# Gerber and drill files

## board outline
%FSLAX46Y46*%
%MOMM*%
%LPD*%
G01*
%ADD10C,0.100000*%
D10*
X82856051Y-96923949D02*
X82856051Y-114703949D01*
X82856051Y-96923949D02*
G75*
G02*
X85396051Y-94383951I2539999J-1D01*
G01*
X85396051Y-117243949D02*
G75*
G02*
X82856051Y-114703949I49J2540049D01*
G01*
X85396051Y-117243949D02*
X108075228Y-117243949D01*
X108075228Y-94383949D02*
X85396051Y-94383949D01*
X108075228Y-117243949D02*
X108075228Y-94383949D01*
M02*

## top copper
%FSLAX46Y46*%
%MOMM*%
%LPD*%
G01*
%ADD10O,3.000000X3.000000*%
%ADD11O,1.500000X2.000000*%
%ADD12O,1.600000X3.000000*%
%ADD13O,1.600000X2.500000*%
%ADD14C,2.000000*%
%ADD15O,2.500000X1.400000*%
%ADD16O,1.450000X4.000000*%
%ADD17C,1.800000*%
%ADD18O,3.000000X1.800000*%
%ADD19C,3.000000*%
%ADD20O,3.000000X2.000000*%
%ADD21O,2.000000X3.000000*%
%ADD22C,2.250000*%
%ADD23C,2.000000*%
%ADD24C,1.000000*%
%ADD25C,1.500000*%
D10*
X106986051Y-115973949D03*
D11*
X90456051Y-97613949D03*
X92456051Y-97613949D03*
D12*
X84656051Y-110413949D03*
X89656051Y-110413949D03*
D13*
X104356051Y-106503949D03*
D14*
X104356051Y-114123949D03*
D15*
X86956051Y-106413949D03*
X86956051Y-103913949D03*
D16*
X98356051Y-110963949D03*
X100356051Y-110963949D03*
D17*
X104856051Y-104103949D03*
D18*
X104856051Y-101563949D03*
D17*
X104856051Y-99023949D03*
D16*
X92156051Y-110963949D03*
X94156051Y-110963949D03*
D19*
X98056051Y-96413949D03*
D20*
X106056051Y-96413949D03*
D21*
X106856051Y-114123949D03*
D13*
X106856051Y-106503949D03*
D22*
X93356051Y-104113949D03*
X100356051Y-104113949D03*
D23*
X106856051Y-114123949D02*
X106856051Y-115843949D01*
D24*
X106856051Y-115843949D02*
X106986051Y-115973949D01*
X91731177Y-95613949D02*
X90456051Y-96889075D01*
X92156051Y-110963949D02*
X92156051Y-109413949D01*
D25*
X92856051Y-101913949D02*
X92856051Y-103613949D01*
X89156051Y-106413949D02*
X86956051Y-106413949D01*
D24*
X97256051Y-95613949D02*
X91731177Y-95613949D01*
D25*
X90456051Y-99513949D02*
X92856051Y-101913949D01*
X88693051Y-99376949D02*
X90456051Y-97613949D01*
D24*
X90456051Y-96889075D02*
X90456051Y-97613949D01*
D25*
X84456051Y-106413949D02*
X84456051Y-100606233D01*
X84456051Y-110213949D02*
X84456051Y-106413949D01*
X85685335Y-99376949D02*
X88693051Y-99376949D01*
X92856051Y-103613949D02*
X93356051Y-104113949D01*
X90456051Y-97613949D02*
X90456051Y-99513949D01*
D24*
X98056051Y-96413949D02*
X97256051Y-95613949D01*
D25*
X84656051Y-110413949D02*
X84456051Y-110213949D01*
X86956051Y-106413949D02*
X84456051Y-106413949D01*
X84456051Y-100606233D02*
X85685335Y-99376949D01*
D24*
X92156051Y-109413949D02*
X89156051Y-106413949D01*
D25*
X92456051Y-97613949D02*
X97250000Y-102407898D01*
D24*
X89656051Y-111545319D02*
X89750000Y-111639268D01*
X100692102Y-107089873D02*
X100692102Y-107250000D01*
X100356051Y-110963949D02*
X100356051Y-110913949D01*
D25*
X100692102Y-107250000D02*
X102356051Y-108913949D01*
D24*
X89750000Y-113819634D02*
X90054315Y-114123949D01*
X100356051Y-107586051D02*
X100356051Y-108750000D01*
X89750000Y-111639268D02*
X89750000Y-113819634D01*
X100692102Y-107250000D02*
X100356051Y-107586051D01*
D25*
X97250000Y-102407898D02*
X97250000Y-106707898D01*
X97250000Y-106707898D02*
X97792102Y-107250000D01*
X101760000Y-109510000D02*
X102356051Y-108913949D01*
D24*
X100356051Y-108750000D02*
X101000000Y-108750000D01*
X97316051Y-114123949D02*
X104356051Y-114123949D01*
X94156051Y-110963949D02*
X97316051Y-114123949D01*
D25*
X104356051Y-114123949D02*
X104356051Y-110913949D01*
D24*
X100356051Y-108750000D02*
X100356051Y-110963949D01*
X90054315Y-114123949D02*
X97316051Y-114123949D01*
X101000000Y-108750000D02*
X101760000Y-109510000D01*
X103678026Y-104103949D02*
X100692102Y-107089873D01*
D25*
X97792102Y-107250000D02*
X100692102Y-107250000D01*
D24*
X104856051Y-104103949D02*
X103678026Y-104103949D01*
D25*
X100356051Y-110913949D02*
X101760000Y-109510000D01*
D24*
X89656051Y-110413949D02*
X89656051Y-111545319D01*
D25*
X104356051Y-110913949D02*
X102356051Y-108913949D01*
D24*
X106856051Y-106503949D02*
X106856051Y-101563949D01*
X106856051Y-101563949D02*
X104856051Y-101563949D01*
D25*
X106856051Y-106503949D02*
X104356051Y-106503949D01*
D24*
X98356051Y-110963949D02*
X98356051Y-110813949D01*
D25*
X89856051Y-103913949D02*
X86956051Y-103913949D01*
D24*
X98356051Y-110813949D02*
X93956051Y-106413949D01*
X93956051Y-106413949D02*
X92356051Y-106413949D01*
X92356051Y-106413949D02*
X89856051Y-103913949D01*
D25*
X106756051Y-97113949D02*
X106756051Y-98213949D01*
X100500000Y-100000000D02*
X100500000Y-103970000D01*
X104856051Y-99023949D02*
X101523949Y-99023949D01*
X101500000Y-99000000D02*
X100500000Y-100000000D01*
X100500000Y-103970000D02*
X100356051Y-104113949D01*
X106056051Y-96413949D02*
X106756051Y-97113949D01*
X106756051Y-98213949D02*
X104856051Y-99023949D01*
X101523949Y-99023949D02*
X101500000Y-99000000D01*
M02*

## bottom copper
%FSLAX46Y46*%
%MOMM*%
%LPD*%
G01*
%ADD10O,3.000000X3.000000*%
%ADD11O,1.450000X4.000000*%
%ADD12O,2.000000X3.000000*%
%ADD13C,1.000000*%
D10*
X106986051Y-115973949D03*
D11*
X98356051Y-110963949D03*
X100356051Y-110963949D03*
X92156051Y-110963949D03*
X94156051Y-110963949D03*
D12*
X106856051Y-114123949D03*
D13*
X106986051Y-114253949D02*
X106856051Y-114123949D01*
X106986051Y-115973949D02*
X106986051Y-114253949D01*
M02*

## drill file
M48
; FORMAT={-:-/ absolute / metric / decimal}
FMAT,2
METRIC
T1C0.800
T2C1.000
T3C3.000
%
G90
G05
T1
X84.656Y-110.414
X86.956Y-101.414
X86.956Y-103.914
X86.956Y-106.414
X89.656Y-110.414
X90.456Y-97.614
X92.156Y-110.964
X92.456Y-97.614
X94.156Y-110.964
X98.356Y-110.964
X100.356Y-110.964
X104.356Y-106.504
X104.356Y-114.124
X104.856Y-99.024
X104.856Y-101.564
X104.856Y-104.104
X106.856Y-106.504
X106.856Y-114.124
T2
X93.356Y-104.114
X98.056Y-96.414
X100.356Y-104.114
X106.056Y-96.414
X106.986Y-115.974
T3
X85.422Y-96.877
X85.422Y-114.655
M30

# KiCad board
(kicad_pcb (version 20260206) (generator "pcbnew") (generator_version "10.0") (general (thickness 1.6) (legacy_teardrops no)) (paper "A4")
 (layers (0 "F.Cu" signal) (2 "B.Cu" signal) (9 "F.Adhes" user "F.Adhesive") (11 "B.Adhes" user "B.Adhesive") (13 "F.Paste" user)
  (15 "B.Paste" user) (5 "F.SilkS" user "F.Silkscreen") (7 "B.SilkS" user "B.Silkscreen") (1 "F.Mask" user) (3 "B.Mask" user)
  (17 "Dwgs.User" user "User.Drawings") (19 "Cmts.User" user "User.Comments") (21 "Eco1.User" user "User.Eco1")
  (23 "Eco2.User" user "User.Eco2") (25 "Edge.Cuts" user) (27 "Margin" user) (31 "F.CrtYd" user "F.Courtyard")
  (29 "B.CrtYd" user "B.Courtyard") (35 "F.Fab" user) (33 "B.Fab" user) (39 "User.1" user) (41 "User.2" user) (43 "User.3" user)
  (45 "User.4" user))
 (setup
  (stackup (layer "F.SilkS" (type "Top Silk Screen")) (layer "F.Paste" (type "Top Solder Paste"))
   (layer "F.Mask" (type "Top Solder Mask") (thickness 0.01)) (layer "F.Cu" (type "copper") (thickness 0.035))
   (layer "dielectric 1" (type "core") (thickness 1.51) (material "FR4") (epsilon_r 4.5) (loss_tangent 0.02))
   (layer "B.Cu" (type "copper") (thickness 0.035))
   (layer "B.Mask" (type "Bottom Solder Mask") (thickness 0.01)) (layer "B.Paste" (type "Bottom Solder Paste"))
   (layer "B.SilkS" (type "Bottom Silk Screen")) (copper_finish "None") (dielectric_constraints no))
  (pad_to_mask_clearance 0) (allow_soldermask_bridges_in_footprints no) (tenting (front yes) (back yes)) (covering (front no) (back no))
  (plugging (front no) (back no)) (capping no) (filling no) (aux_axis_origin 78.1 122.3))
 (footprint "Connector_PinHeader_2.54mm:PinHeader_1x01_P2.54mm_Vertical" (layer "F.Cu") (at 106.986051 115.973949 180)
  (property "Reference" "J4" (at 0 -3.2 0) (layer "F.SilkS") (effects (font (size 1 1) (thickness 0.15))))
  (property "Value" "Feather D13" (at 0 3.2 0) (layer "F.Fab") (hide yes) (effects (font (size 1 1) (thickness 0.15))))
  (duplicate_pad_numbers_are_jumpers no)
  (pad "e" thru_hole oval (at 0 0 180) (size 3 3) (drill 1) (layers "*.Cu" "F.Mask") (remove_unused_layers no) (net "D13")))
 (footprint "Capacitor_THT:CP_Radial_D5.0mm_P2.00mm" (layer "F.Cu") (at 91.456051 97.613949)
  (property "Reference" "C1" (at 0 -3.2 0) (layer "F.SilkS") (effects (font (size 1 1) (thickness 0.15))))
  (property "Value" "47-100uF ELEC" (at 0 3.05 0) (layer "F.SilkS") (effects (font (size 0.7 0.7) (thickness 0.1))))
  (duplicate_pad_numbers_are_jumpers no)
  (pad "1" thru_hole oval (at -1 0) (size 1.5 2) (drill 0.8) (layers "*.Cu" "F.Mask") (remove_unused_layers yes) (keep_end_layers no)
   (zone_layer_connections) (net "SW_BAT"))
  (pad "2" thru_hole oval (at 1 0) (size 1.5 2) (drill 0.8) (layers "*.Cu" "F.Mask") (remove_unused_layers yes) (keep_end_layers no)
   (zone_layer_connections) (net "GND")))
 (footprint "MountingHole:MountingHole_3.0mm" (layer "F.Cu") (at 85.422051 96.876949 180)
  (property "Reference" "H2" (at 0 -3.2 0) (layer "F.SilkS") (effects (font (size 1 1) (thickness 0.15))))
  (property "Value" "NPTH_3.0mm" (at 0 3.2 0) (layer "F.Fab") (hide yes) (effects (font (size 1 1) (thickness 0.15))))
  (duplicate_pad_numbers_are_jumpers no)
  (pad "" np_thru_hole circle (at 0 0 180) (size 3 3) (drill 3) (layers "*.Cu" "*.Mask")))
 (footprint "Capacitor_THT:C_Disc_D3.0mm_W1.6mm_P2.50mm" (layer "F.Cu") (at 87.156051 110.413949)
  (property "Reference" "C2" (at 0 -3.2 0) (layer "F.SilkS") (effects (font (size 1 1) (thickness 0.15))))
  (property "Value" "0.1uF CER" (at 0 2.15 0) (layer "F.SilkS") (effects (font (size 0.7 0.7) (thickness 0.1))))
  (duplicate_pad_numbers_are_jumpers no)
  (pad "1" thru_hole oval (at -2.5 0) (size 1.6 3) (drill 0.8) (layers "*.Cu" "F.Mask") (remove_unused_layers yes) (keep_end_layers no)
   (zone_layer_connections) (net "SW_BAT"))
  (pad "2" thru_hole oval (at 2.5 0) (size 1.6 3) (drill 0.8) (layers "*.Cu" "F.Mask") (remove_unused_layers yes) (keep_end_layers no)
   (zone_layer_connections) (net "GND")))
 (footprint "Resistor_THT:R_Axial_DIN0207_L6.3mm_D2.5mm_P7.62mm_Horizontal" (layer "F.Cu") (at 104.356051 110.313949 -90)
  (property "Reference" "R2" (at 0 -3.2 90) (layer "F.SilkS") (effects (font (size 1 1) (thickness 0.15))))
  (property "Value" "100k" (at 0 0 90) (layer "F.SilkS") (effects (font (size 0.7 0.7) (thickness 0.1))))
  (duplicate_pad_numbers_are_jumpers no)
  (pad "1" thru_hole oval (at -3.81 0 270) (size 2.5 1.6) (drill 0.8) (layers "*.Cu" "F.Mask") (remove_unused_layers yes)
   (keep_end_layers no) (zone_layer_connections) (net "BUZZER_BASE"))
  (pad "2" thru_hole circle (at 3.81 0 270) (size 2 2) (drill 0.8) (layers "*.Cu" "F.Mask") (remove_unused_layers yes) (keep_end_layers no)
   (zone_layer_connections) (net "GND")))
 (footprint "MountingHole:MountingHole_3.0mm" (layer "F.Cu") (at 85.422051 114.655349 180)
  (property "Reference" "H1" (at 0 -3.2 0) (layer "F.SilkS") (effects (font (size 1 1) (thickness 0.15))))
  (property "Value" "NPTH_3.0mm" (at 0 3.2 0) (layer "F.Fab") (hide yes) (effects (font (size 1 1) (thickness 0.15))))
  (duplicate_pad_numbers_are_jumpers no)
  (pad "" np_thru_hole circle (at 0 0 180) (size 3 3) (drill 3) (layers "*.Cu" "*.Mask")))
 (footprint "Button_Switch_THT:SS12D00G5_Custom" (layer "F.Cu") (at 86.956051 103.913949 90)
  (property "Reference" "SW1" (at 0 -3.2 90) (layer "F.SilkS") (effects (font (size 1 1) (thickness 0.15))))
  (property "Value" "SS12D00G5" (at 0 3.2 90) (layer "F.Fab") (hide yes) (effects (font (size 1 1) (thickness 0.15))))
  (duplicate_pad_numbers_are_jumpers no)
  (pad "1" thru_hole oval (at -2.5 0 90) (size 1.4 2.5) (drill 0.8) (layers "*.Cu" "F.Mask") (remove_unused_layers yes) (keep_end_layers no)
   (zone_layer_connections) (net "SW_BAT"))
  (pad "2" thru_hole oval (at 0 0 90) (size 1.4 2.5) (drill 0.8) (layers "*.Cu" "F.Mask") (remove_unused_layers yes) (keep_end_layers no)
   (zone_layer_connections) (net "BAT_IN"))
  (pad "3" thru_hole oval (at 2.5 0 90) (size 1.4 2.5) (drill 0.8) (layers "*.Cu" "F.Mask") (remove_unused_layers yes) (keep_end_layers no)
   (zone_layer_connections)))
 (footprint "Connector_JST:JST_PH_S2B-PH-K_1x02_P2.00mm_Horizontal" (layer "F.Cu") (at 99.356051 112.713949)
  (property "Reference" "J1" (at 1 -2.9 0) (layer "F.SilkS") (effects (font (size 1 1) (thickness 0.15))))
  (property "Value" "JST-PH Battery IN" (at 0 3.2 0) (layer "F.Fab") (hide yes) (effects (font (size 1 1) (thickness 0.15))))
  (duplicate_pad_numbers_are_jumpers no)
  (pad "1" thru_hole oval (at -1 -1.75) (size 1.45 4) (drill 0.8) (layers "*.Cu" "F.Mask") (remove_unused_layers no) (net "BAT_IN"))
  (pad "2" thru_hole oval (at 1 -1.75) (size 1.45 4) (drill 0.8) (layers "*.Cu" "F.Mask") (remove_unused_layers no) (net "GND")))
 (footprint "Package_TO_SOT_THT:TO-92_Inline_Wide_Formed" (layer "F.Cu") (at 104.856051 101.563949 90)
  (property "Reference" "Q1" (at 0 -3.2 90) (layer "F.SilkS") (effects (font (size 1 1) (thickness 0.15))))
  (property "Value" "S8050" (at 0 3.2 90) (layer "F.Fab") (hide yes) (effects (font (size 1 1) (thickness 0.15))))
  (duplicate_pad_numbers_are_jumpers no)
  (pad "1" thru_hole circle (at -2.54 0 90) (size 1.8 1.8) (drill 0.8) (layers "*.Cu" "F.Mask") (remove_unused_layers yes)
   (keep_end_layers no) (zone_layer_connections) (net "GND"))
  (pad "2" thru_hole oval (at 0 0 90) (size 1.8 3) (drill 0.8) (layers "*.Cu" "F.Mask") (remove_unused_layers yes) (keep_end_layers no)
   (zone_layer_connections) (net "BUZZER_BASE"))
  (pad "3" thru_hole circle (at 2.54 0 90) (size 1.8 1.8) (drill 0.8) (layers "*.Cu" "F.Mask") (remove_unused_layers yes)
   (keep_end_layers no) (zone_layer_connections) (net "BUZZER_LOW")))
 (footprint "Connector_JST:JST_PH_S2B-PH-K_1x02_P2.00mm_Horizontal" (layer "F.Cu") (at 93.156051 112.713949)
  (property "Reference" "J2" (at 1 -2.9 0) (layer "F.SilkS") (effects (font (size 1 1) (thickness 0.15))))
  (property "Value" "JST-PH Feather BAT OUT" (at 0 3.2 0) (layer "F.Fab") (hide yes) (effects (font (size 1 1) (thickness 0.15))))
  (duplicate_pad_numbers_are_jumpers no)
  (pad "1" thru_hole oval (at -1 -1.75) (size 1.45 4) (drill 0.8) (layers "*.Cu" "F.Mask") (remove_unused_layers no) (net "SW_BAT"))
  (pad "2" thru_hole oval (at 1 -1.75) (size 1.45 4) (drill 0.8) (layers "*.Cu" "F.Mask") (remove_unused_layers no) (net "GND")))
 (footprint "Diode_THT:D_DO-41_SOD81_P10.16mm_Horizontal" (layer "F.Cu") (at 102.056051 96.413949)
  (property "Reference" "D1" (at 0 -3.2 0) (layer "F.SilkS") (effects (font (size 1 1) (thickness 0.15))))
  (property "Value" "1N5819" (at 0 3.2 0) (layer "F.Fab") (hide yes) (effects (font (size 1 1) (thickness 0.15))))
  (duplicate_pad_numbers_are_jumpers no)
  (pad "1" thru_hole circle (at -4 0) (size 3 3) (drill 1) (layers "*.Cu" "F.Mask") (remove_unused_layers yes) (keep_end_layers no)
   (zone_layer_connections) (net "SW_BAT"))
  (pad "2" thru_hole oval (at 4 0) (size 3 2) (drill 1) (layers "*.Cu" "F.Mask") (remove_unused_layers yes) (keep_end_layers no)
   (zone_layer_connections) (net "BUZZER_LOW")))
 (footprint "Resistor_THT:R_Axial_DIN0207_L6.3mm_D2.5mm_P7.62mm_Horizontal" (layer "F.Cu") (at 106.856051 110.313949 90)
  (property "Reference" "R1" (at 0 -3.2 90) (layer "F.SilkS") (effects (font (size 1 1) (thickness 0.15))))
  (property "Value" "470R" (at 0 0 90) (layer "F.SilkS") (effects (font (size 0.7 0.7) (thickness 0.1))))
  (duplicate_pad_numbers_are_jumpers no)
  (pad "1" thru_hole oval (at -3.81 0 90) (size 3 2) (drill 0.8) (layers "*.Cu" "F.Mask") (remove_unused_layers no) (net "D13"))
  (pad "2" thru_hole oval (at 3.81 0 90) (size 2.5 1.6) (drill 0.8) (layers "*.Cu" "F.Mask") (remove_unused_layers yes) (keep_end_layers no)
   (zone_layer_connections) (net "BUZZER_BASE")))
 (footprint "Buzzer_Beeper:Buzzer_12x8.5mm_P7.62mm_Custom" (layer "F.Cu") (at 96.856051 104.113949)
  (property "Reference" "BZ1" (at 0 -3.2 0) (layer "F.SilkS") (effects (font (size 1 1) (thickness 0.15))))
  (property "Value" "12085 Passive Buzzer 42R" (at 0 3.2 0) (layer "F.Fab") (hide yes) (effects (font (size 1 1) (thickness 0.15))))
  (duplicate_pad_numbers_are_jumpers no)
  (pad "1" thru_hole circle (at -3.5 0) (size 2.25 2.25) (drill 1) (layers "*.Cu" "F.Mask") (remove_unused_layers yes) (keep_end_layers no)
   (zone_layer_connections) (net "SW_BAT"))
  (pad "2" thru_hole circle (at 3.5 0) (size 2.25 2.25) (drill 1) (layers "*.Cu" "F.Mask") (remove_unused_layers yes) (keep_end_layers no)
   (zone_layer_connections) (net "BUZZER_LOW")))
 (gr_line (start 82.856051 96.923949) (end 82.856051 114.703949) (stroke (width 0.1) (type default)) (layer "Edge.Cuts"))
 (gr_arc (start 82.856051 96.923949) (mid 83.6 95.127898) (end 85.396051 94.383949) (stroke (width 0.1) (type default)) (layer "Edge.Cuts"))
 (gr_arc (start 85.396051 117.243949) (mid 83.6 116.5) (end 82.856051 114.703949) (stroke (width 0.1) (type default)) (layer "Edge.Cuts"))
 (gr_line (start 85.396051 117.243949) (end 108.075228 117.243949) (stroke (width 0.1) (type default)) (layer "Edge.Cuts"))
 (gr_line (start 108.075228 94.383949) (end 85.396051 94.383949) (stroke (width 0.1) (type default)) (layer "Edge.Cuts"))
 (gr_line (start 108.075228 117.243949) (end 108.075228 94.383949) (stroke (width 0.1) (type default)) (layer "Edge.Cuts"))
 (segment (start 106.856051 114.123949) (end 106.856051 115.843949) (width 2) (layer "F.Cu") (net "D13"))
 (segment (start 106.856051 115.843949) (end 106.986051 115.973949) (width 1) (layer "F.Cu") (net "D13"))
 (segment (start 106.986051 114.253949) (end 106.856051 114.123949) (width 1) (layer "B.Cu") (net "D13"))
 (segment (start 106.986051 115.973949) (end 106.986051 114.253949) (width 1) (layer "B.Cu") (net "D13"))
 (segment (start 91.731177 95.613949) (end 90.456051 96.889075) (width 1) (layer "F.Cu") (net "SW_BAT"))
 (segment (start 92.156051 110.963949) (end 92.156051 109.413949) (width 1) (layer "F.Cu") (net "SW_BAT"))
 (segment (start 92.856051 101.913949) (end 92.856051 103.613949) (width 1.5) (layer "F.Cu") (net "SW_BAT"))
 (segment (start 89.156051 106.413949) (end 86.956051 106.413949) (width 1.5) (layer "F.Cu") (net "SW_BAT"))
 (segment (start 97.256051 95.613949) (end 91.731177 95.613949) (width 1) (layer "F.Cu") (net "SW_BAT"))
 (segment (start 90.456051 99.513949) (end 92.856051 101.913949) (width 1.5) (layer "F.Cu") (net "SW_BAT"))
 (segment (start 88.693051 99.376949) (end 90.456051 97.613949) (width 1.5) (layer "F.Cu") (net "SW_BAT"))
 (segment (start 90.456051 96.889075) (end 90.456051 97.613949) (width 1) (layer "F.Cu") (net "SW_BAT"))
 (segment (start 84.456051 106.413949) (end 84.456051 100.606233) (width 1.5) (layer "F.Cu") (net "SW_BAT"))
 (segment (start 84.456051 110.213949) (end 84.456051 106.413949) (width 1.5) (layer "F.Cu") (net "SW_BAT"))
 (segment (start 85.685335 99.376949) (end 88.693051 99.376949) (width 1.5) (layer "F.Cu") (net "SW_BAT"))
 (segment (start 92.856051 103.613949) (end 93.356051 104.113949) (width 1.5) (layer "F.Cu") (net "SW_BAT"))
 (segment (start 90.456051 97.613949) (end 90.456051 99.513949) (width 1.5) (layer "F.Cu") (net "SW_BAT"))
 (segment (start 98.056051 96.413949) (end 97.256051 95.613949) (width 1) (layer "F.Cu") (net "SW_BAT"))
 (segment (start 84.656051 110.413949) (end 84.456051 110.213949) (width 1.5) (layer "F.Cu") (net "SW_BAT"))
 (segment (start 86.956051 106.413949) (end 84.456051 106.413949) (width 1.5) (layer "F.Cu") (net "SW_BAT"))
 (segment (start 84.456051 100.606233) (end 85.685335 99.376949) (width 1.5) (layer "F.Cu") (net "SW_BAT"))
 (segment (start 92.156051 109.413949) (end 89.156051 106.413949) (width 1) (layer "F.Cu") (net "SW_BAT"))
 (segment (start 92.456051 97.613949) (end 97.25 102.407898) (width 1.5) (layer "F.Cu") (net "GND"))
 (segment (start 89.656051 111.545319) (end 89.75 111.639268) (width 1) (layer "F.Cu") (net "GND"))
 (segment (start 100.692102 107.089873) (end 100.692102 107.25) (width 1) (layer "F.Cu") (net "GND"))
 (segment (start 100.356051 110.963949) (end 100.356051 110.913949) (width 1) (layer "F.Cu") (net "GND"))
 (segment (start 100.692102 107.25) (end 102.356051 108.913949) (width 1.5) (layer "F.Cu") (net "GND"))
 (segment (start 89.75 113.819634) (end 90.054315 114.123949) (width 1) (layer "F.Cu") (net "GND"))
 (segment (start 100.356051 107.586051) (end 100.356051 108.75) (width 1) (layer "F.Cu") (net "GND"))
 (segment (start 89.75 111.639268) (end 89.75 113.819634) (width 1) (layer "F.Cu") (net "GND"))
 (segment (start 100.692102 107.25) (end 100.356051 107.586051) (width 1) (layer "F.Cu") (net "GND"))
 (segment (start 97.25 102.407898) (end 97.25 106.707898) (width 1.5) (layer "F.Cu") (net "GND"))
 (segment (start 97.25 106.707898) (end 97.792102 107.25) (width 1.5) (layer "F.Cu") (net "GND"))
 (segment (start 101.76 109.51) (end 102.356051 108.913949) (width 1.5) (layer "F.Cu") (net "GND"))
 (segment (start 100.356051 108.75) (end 101 108.75) (width 1) (layer "F.Cu") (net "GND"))
 (segment (start 97.316051 114.123949) (end 104.356051 114.123949) (width 1) (layer "F.Cu") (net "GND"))
 (segment (start 94.156051 110.963949) (end 97.316051 114.123949) (width 1) (layer "F.Cu") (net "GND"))
 (segment (start 104.356051 114.123949) (end 104.356051 110.913949) (width 1.5) (layer "F.Cu") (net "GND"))
 (segment (start 100.356051 108.75) (end 100.356051 110.963949) (width 1) (layer "F.Cu") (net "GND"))
 (segment (start 90.054315 114.123949) (end 97.316051 114.123949) (width 1) (layer "F.Cu") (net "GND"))
 (segment (start 101 108.75) (end 101.76 109.51) (width 1) (layer "F.Cu") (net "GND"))
 (segment (start 103.678026 104.103949) (end 100.692102 107.089873) (width 1) (layer "F.Cu") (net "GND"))
 (segment (start 97.792102 107.25) (end 100.692102 107.25) (width 1.5) (layer "F.Cu") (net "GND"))
 (segment (start 104.856051 104.103949) (end 103.678026 104.103949) (width 1) (layer "F.Cu") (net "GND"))
 (segment (start 100.356051 110.913949) (end 101.76 109.51) (width 1.5) (layer "F.Cu") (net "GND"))
 (segment (start 89.656051 110.413949) (end 89.656051 111.545319) (width 1) (layer "F.Cu") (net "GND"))
 (segment (start 104.356051 110.913949) (end 102.356051 108.913949) (width 1.5) (layer "F.Cu") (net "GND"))
 (segment (start 106.856051 106.503949) (end 106.856051 101.563949) (width 1) (layer "F.Cu") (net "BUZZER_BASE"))
 (segment (start 106.856051 101.563949) (end 104.856051 101.563949) (width 1) (layer "F.Cu") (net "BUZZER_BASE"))
 (segment (start 106.856051 106.503949) (end 104.356051 106.503949) (width 1.5) (layer "F.Cu") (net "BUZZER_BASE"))
 (segment (start 98.356051 110.963949) (end 98.356051 110.813949) (width 1) (layer "F.Cu") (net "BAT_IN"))
 (segment (start 89.856051 103.913949) (end 86.956051 103.913949) (width 1.5) (layer "F.Cu") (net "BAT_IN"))
 (segment (start 98.356051 110.813949) (end 93.956051 106.413949) (width 1) (layer "F.Cu") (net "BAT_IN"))
 (segment (start 93.956051 106.413949) (end 92.356051 106.413949) (width 1) (layer "F.Cu") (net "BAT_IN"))
 (segment (start 92.356051 106.413949) (end 89.856051 103.913949) (width 1) (layer "F.Cu") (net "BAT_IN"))
 (segment (start 106.756051 97.113949) (end 106.756051 98.213949) (width 1.5) (layer "F.Cu") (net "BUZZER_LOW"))
 (segment (start 100.5 100) (end 100.5 103.97) (width 1.5) (layer "F.Cu") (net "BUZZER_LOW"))
 (segment (start 104.856051 99.023949) (end 101.523949 99.023949) (width 1.5) (layer "F.Cu") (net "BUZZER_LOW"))
 (segment (start 101.5 99) (end 100.5 100) (width 1.5) (layer "F.Cu") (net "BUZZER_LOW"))
 (segment (start 100.5 103.97) (end 100.356051 104.113949) (width 1.5) (layer "F.Cu") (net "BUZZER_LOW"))
 (segment (start 106.056051 96.413949) (end 106.756051 97.113949) (width 1.5) (layer "F.Cu") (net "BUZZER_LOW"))
 (segment (start 106.756051 98.213949) (end 104.856051 99.023949) (width 1.5) (layer "F.Cu") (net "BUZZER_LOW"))
 (segment (start 101.523949 99.023949) (end 101.5 99) (width 1.5) (layer "F.Cu") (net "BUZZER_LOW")))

